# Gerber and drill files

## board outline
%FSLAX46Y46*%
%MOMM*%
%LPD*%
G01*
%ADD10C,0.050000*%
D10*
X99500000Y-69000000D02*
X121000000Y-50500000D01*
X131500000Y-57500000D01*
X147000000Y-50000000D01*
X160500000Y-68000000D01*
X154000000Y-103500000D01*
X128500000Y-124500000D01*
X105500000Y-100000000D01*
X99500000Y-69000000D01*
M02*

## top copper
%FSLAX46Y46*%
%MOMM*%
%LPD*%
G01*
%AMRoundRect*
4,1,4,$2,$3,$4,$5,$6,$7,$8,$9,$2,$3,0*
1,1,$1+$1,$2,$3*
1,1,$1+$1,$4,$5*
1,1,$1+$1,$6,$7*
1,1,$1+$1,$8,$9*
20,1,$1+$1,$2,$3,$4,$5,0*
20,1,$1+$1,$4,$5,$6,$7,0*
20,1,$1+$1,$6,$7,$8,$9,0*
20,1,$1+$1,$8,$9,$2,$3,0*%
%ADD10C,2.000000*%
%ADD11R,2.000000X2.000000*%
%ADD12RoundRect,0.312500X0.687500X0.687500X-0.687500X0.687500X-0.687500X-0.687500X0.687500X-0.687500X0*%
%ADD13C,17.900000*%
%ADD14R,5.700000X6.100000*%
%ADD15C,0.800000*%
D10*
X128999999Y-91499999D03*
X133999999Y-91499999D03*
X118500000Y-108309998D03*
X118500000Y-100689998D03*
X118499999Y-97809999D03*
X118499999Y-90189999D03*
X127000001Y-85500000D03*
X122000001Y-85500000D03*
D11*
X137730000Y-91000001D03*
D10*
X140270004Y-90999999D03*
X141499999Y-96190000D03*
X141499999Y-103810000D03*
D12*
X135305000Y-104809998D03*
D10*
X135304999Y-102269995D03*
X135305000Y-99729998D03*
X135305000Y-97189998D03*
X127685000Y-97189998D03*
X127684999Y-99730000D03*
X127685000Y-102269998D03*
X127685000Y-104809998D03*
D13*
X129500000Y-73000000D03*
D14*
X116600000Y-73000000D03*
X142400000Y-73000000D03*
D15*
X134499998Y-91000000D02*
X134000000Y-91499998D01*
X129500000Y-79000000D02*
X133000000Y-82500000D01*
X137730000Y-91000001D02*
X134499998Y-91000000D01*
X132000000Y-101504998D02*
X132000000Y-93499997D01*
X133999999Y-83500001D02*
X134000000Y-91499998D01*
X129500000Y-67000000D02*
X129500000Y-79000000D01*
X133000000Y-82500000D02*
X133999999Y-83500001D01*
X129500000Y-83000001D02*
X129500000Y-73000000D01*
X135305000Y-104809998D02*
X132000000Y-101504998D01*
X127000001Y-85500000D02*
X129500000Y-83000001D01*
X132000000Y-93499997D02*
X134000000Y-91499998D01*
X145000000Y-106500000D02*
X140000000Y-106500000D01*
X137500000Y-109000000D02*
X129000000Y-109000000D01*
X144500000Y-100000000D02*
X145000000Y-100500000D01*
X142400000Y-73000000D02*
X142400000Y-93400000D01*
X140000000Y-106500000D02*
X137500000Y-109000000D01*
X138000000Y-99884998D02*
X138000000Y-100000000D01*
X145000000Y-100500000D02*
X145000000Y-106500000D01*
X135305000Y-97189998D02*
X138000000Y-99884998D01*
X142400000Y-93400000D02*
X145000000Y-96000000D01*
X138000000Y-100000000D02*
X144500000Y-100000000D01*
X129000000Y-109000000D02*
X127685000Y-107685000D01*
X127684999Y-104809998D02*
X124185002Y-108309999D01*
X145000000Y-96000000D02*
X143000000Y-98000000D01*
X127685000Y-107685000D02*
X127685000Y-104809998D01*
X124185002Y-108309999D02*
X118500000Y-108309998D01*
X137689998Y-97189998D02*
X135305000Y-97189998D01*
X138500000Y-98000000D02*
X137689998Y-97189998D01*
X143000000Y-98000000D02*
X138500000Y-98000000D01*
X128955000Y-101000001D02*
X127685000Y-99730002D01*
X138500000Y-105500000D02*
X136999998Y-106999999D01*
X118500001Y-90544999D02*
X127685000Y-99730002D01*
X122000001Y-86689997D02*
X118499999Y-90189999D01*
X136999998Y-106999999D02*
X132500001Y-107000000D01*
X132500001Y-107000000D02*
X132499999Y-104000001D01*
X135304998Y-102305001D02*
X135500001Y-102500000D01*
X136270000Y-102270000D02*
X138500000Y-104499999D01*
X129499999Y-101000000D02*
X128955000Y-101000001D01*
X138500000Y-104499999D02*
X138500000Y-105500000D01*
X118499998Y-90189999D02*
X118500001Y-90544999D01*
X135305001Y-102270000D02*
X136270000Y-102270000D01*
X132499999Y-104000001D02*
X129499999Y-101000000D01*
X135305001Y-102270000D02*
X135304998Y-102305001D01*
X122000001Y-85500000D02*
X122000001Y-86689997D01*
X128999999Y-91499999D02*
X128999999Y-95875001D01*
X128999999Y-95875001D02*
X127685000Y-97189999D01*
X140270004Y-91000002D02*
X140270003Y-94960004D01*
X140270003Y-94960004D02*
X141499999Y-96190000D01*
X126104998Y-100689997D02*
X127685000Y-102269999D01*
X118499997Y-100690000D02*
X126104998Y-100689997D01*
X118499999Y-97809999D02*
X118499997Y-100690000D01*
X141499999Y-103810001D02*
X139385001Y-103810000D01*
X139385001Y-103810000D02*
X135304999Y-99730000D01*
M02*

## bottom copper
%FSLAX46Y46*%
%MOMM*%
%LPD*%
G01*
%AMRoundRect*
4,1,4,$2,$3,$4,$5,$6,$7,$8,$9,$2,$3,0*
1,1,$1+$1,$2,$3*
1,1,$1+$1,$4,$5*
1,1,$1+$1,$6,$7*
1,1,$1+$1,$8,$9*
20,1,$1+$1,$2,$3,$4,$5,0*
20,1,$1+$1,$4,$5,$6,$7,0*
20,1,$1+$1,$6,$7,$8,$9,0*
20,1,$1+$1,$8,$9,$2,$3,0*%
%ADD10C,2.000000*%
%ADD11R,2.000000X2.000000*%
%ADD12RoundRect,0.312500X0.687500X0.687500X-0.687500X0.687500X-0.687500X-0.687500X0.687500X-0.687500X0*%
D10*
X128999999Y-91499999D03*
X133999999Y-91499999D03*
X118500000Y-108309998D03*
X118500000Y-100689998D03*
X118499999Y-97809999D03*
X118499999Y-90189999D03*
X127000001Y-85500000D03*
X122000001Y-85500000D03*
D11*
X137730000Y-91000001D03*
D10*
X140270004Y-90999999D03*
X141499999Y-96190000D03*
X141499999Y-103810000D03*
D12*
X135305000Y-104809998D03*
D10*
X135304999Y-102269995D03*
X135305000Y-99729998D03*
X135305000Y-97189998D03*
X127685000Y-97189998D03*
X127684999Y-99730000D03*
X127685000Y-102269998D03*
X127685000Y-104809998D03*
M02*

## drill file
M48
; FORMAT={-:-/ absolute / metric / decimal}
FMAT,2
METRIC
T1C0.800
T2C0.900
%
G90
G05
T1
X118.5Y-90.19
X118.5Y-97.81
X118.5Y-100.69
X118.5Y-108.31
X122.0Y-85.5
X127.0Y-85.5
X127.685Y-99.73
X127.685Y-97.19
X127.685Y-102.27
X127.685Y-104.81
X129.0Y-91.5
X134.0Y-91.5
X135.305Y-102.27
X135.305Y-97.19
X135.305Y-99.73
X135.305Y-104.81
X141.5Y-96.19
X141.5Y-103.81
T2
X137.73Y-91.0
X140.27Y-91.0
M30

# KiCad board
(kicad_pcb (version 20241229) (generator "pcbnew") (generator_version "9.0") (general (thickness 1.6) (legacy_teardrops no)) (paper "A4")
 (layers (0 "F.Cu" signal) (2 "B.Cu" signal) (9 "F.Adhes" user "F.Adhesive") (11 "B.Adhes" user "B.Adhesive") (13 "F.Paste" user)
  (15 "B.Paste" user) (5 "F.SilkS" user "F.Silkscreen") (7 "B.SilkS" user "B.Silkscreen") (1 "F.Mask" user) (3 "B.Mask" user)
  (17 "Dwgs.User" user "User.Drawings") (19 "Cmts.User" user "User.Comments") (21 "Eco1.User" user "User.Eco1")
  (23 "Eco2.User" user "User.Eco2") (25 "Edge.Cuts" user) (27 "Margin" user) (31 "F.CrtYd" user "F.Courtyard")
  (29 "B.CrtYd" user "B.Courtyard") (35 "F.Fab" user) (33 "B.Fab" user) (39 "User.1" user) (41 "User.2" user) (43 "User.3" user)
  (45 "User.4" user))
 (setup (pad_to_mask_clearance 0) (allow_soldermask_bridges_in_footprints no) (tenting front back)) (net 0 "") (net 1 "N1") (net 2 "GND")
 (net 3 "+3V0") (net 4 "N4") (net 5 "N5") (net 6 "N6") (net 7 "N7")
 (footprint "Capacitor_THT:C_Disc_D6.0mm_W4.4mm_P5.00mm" (layer "F.Cu") (at 128.999999 91.499999)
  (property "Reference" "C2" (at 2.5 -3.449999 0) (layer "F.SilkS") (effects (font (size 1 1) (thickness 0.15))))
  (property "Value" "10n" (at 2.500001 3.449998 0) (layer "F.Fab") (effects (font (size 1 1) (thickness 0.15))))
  (pad "1" thru_hole circle (at 0 0) (size 2 2) (drill 0.8) (layers "*.Cu" "*.Mask") (remove_unused_layers no) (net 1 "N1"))
  (pad "2" thru_hole circle (at 5 0) (size 2 2) (drill 0.8) (layers "*.Cu" "*.Mask") (remove_unused_layers no) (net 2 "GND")))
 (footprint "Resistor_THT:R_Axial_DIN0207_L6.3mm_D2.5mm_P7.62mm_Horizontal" (layer "F.Cu") (at 118.5 108.309998 90)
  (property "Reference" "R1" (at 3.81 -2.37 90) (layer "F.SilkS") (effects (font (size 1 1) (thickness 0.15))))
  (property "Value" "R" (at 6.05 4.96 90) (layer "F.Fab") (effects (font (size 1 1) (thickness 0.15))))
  (pad "1" thru_hole circle (at 0 0 90) (size 2 2) (drill 0.8) (layers "*.Cu" "*.Mask") (remove_unused_layers no) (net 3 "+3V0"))
  (pad "2" thru_hole circle (at 7.62 0 90) (size 2 2) (drill 0.8) (layers "*.Cu" "*.Mask") (remove_unused_layers no) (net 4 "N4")))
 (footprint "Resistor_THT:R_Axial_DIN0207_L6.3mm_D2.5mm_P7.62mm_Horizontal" (layer "F.Cu") (at 118.499999 97.809999 90)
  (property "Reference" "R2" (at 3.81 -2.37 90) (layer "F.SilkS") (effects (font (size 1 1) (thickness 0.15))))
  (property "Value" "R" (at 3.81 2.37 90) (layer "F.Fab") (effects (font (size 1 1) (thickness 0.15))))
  (pad "1" thru_hole circle (at 0 0 90) (size 2 2) (drill 0.8) (layers "*.Cu" "*.Mask") (remove_unused_layers no) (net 4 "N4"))
  (pad "2" thru_hole circle (at 7.62 0 90) (size 2 2) (drill 0.8) (layers "*.Cu" "*.Mask") (remove_unused_layers no) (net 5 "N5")))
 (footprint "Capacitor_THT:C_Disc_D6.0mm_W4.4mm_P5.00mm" (layer "F.Cu") (at 127.000001 85.5 180)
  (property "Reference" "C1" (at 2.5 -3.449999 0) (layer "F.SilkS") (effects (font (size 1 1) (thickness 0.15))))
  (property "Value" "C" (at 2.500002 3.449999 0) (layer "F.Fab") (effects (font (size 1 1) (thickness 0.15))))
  (pad "1" thru_hole circle (at 0 0 180) (size 2 2) (drill 0.8) (layers "*.Cu" "*.Mask") (remove_unused_layers no) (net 2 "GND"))
  (pad "2" thru_hole circle (at 5 0 180) (size 2 2) (drill 0.8) (layers "*.Cu" "*.Mask") (remove_unused_layers no) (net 5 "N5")))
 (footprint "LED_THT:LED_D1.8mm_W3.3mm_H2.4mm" (layer "F.Cu") (at 137.73 91.000001)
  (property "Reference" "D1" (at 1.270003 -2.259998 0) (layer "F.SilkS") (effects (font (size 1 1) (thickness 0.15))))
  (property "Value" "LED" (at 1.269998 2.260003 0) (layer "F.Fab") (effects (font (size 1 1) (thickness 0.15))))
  (pad "1" thru_hole rect (at 0 0) (size 2 2) (drill 0.9) (layers "*.Cu" "*.Mask") (remove_unused_layers no) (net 2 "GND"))
  (pad "2" thru_hole circle (at 2.540004 -0.000002) (size 2 2) (drill 0.9) (layers "*.Cu" "*.Mask") (remove_unused_layers no) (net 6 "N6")))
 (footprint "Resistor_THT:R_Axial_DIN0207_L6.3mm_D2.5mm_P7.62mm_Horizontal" (layer "F.Cu") (at 141.499999 96.19 -90)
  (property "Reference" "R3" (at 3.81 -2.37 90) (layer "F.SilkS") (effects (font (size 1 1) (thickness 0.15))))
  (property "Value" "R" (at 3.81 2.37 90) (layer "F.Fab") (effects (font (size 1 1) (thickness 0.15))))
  (pad "1" thru_hole circle (at 0 0 270) (size 2 2) (drill 0.8) (layers "*.Cu" "*.Mask") (remove_unused_layers no) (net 6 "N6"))
  (pad "2" thru_hole circle (at 7.62 0 270) (size 2 2) (drill 0.8) (layers "*.Cu" "*.Mask") (remove_unused_layers no) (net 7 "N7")))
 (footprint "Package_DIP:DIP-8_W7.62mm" (layer "F.Cu") (at 135.305 104.809998 180)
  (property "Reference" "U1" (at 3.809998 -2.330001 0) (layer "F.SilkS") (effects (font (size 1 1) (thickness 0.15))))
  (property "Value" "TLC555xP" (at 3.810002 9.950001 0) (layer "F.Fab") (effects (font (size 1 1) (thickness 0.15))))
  (pad "1" thru_hole roundrect (at 0 0 180) (size 2 2) (drill 0.8) (layers "*.Cu" "*.Mask") (remove_unused_layers no)
   (roundrect_rratio 0.15625) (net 2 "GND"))
  (pad "2" thru_hole circle (at 0.000001 2.540003 180) (size 2 2) (drill 0.8) (layers "*.Cu" "*.Mask") (remove_unused_layers no)
   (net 5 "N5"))
  (pad "3" thru_hole circle (at 0 5.08 180) (size 2 2) (drill 0.8) (layers "*.Cu" "*.Mask") (remove_unused_layers no) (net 7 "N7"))
  (pad "4" thru_hole circle (at 0 7.62 180) (size 2 2) (drill 0.8) (layers "*.Cu" "*.Mask") (remove_unused_layers no) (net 3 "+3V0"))
  (pad "5" thru_hole circle (at 7.62 7.62 180) (size 2 2) (drill 0.8) (layers "*.Cu" "*.Mask") (remove_unused_layers no) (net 1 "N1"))
  (pad "6" thru_hole circle (at 7.620001 5.079998 180) (size 2 2) (drill 0.8) (layers "*.Cu" "*.Mask") (remove_unused_layers no)
   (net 5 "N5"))
  (pad "7" thru_hole circle (at 7.62 2.54 180) (size 2 2) (drill 0.8) (layers "*.Cu" "*.Mask") (remove_unused_layers no) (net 4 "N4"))
  (pad "8" thru_hole circle (at 7.62 0 180) (size 2 2) (drill 0.8) (layers "*.Cu" "*.Mask") (remove_unused_layers no) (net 3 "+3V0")))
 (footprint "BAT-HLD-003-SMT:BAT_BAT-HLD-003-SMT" (layer "F.Cu") (at 129.5 73)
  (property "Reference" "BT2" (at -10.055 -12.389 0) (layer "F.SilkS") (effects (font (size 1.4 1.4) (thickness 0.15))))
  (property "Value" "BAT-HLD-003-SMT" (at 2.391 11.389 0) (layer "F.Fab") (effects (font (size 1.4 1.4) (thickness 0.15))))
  (pad "N" smd circle (at 0 0) (size 17.9 17.9) (layers "F.Cu" "F.Mask") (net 2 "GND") (solder_mask_margin 0.102))
  (pad "P1" smd rect (at -12.9 0) (size 5.7 6.1) (layers "F.Cu" "F.Mask" "F.Paste") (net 3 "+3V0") (solder_mask_margin 0.102))
  (pad "P2" smd rect (at 12.9 0) (size 5.7 6.1) (layers "F.Cu" "F.Mask" "F.Paste") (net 3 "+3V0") (solder_mask_margin 0.102)))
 (gr_poly
  (pts (xy 99.5 69) (xy 121 50.5) (xy 131.5 57.5) (xy 147 50) (xy 160.5 68) (xy 154 103.5) (xy 128.5 124.5) (xy 105.5 100))
  (stroke (width 0.05) (type solid)) (fill no) (layer "Edge.Cuts"))
 (segment (start 134.499998 91) (end 134 91.499998) (width 0.8) (layer "F.Cu") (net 2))
 (segment (start 129.5 79) (end 133 82.5) (width 0.8) (layer "F.Cu") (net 2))
 (segment (start 137.73 91.000001) (end 134.499998 91) (width 0.8) (layer "F.Cu") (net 2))
 (segment (start 132 101.504998) (end 132 93.499997) (width 0.8) (layer "F.Cu") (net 2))
 (segment (start 133.999999 83.500001) (end 134 91.499998) (width 0.8) (layer "F.Cu") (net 2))
 (segment (start 129.5 67) (end 129.5 79) (width 0.8) (layer "F.Cu") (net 2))
 (segment (start 133 82.5) (end 133.999999 83.500001) (width 0.8) (layer "F.Cu") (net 2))
 (segment (start 129.5 83.000001) (end 129.5 73) (width 0.8) (layer "F.Cu") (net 2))
 (segment (start 135.305 104.809998) (end 132 101.504998) (width 0.8) (layer "F.Cu") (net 2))
 (segment (start 127.000001 85.5) (end 129.5 83.000001) (width 0.8) (layer "F.Cu") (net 2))
 (segment (start 132 93.499997) (end 134 91.499998) (width 0.8) (layer "F.Cu") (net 2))
 (segment (start 145 106.5) (end 140 106.5) (width 0.8) (layer "F.Cu") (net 3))
 (segment (start 137.5 109) (end 129 109) (width 0.8) (layer "F.Cu") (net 3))
 (segment (start 144.5 100) (end 145 100.5) (width 0.8) (layer "F.Cu") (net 3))
 (segment (start 142.4 73) (end 142.4 93.4) (width 0.8) (layer "F.Cu") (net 3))
 (segment (start 140 106.5) (end 137.5 109) (width 0.8) (layer "F.Cu") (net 3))
 (segment (start 138 99.884998) (end 138 100) (width 0.8) (layer "F.Cu") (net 3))
 (segment (start 145 100.5) (end 145 106.5) (width 0.8) (layer "F.Cu") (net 3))
 (segment (start 135.305 97.189998) (end 138 99.884998) (width 0.8) (layer "F.Cu") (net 3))
 (segment (start 142.4 93.4) (end 145 96) (width 0.8) (layer "F.Cu") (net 3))
 (segment (start 138 100) (end 144.5 100) (width 0.8) (layer "F.Cu") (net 3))
 (segment (start 129 109) (end 127.685 107.685) (width 0.8) (layer "F.Cu") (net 3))
 (segment (start 127.684999 104.809998) (end 124.185002 108.309999) (width 0.8) (layer "F.Cu") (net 3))
 (segment (start 145 96) (end 143 98) (width 0.8) (layer "F.Cu") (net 3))
 (segment (start 127.685 107.685) (end 127.685 104.809998) (width 0.8) (layer "F.Cu") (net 3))
 (segment (start 124.185002 108.309999) (end 118.5 108.309998) (width 0.8) (layer "F.Cu") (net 3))
 (segment (start 137.689998 97.189998) (end 135.305 97.189998) (width 0.8) (layer "F.Cu") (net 3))
 (segment (start 138.5 98) (end 137.689998 97.189998) (width 0.8) (layer "F.Cu") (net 3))
 (segment (start 143 98) (end 138.5 98) (width 0.8) (layer "F.Cu") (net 3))
 (segment (start 128.955 101.000001) (end 127.685 99.730002) (width 0.8) (layer "F.Cu") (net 5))
 (segment (start 138.5 105.5) (end 136.999998 106.999999) (width 0.8) (layer "F.Cu") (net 5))
 (segment (start 118.500001 90.544999) (end 127.685 99.730002) (width 0.8) (layer "F.Cu") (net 5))
 (segment (start 122.000001 86.689997) (end 118.499999 90.189999) (width 0.8) (layer "F.Cu") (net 5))
 (segment (start 136.999998 106.999999) (end 132.500001 107) (width 0.8) (layer "F.Cu") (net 5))
 (segment (start 132.500001 107) (end 132.499999 104.000001) (width 0.8) (layer "F.Cu") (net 5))
 (segment (start 135.304998 102.305001) (end 135.500001 102.5) (width 0.8) (layer "F.Cu") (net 5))
 (segment (start 136.27 102.27) (end 138.5 104.499999) (width 0.8) (layer "F.Cu") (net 5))
 (segment (start 129.499999 101) (end 128.955 101.000001) (width 0.8) (layer "F.Cu") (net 5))
 (segment (start 138.5 104.499999) (end 138.5 105.5) (width 0.8) (layer "F.Cu") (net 5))
 (segment (start 118.499998 90.189999) (end 118.500001 90.544999) (width 0.8) (layer "F.Cu") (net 5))
 (segment (start 135.305001 102.27) (end 136.27 102.27) (width 0.8) (layer "F.Cu") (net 5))
 (segment (start 132.499999 104.000001) (end 129.499999 101) (width 0.8) (layer "F.Cu") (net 5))
 (segment (start 135.305001 102.27) (end 135.304998 102.305001) (width 0.8) (layer "F.Cu") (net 5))
 (segment (start 122.000001 85.5) (end 122.000001 86.689997) (width 0.8) (layer "F.Cu") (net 5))
 (segment (start 128.999999 91.499999) (end 128.999999 95.875001) (width 0.8) (layer "F.Cu") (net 1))
 (segment (start 128.999999 95.875001) (end 127.685 97.189999) (width 0.8) (layer "F.Cu") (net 1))
 (segment (start 140.270004 91.000002) (end 140.270003 94.960004) (width 0.8) (layer "F.Cu") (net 6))
 (segment (start 140.270003 94.960004) (end 141.499999 96.19) (width 0.8) (layer "F.Cu") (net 6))
 (segment (start 126.104998 100.689997) (end 127.685 102.269999) (width 0.8) (layer "F.Cu") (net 4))
 (segment (start 118.499997 100.69) (end 126.104998 100.689997) (width 0.8) (layer "F.Cu") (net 4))
 (segment (start 118.499999 97.809999) (end 118.499997 100.69) (width 0.8) (layer "F.Cu") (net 4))
 (segment (start 141.499999 103.810001) (end 139.385001 103.81) (width 0.8) (layer "F.Cu") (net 7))
 (segment (start 139.385001 103.81) (end 135.304999 99.73) (width 0.8) (layer "F.Cu") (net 7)))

